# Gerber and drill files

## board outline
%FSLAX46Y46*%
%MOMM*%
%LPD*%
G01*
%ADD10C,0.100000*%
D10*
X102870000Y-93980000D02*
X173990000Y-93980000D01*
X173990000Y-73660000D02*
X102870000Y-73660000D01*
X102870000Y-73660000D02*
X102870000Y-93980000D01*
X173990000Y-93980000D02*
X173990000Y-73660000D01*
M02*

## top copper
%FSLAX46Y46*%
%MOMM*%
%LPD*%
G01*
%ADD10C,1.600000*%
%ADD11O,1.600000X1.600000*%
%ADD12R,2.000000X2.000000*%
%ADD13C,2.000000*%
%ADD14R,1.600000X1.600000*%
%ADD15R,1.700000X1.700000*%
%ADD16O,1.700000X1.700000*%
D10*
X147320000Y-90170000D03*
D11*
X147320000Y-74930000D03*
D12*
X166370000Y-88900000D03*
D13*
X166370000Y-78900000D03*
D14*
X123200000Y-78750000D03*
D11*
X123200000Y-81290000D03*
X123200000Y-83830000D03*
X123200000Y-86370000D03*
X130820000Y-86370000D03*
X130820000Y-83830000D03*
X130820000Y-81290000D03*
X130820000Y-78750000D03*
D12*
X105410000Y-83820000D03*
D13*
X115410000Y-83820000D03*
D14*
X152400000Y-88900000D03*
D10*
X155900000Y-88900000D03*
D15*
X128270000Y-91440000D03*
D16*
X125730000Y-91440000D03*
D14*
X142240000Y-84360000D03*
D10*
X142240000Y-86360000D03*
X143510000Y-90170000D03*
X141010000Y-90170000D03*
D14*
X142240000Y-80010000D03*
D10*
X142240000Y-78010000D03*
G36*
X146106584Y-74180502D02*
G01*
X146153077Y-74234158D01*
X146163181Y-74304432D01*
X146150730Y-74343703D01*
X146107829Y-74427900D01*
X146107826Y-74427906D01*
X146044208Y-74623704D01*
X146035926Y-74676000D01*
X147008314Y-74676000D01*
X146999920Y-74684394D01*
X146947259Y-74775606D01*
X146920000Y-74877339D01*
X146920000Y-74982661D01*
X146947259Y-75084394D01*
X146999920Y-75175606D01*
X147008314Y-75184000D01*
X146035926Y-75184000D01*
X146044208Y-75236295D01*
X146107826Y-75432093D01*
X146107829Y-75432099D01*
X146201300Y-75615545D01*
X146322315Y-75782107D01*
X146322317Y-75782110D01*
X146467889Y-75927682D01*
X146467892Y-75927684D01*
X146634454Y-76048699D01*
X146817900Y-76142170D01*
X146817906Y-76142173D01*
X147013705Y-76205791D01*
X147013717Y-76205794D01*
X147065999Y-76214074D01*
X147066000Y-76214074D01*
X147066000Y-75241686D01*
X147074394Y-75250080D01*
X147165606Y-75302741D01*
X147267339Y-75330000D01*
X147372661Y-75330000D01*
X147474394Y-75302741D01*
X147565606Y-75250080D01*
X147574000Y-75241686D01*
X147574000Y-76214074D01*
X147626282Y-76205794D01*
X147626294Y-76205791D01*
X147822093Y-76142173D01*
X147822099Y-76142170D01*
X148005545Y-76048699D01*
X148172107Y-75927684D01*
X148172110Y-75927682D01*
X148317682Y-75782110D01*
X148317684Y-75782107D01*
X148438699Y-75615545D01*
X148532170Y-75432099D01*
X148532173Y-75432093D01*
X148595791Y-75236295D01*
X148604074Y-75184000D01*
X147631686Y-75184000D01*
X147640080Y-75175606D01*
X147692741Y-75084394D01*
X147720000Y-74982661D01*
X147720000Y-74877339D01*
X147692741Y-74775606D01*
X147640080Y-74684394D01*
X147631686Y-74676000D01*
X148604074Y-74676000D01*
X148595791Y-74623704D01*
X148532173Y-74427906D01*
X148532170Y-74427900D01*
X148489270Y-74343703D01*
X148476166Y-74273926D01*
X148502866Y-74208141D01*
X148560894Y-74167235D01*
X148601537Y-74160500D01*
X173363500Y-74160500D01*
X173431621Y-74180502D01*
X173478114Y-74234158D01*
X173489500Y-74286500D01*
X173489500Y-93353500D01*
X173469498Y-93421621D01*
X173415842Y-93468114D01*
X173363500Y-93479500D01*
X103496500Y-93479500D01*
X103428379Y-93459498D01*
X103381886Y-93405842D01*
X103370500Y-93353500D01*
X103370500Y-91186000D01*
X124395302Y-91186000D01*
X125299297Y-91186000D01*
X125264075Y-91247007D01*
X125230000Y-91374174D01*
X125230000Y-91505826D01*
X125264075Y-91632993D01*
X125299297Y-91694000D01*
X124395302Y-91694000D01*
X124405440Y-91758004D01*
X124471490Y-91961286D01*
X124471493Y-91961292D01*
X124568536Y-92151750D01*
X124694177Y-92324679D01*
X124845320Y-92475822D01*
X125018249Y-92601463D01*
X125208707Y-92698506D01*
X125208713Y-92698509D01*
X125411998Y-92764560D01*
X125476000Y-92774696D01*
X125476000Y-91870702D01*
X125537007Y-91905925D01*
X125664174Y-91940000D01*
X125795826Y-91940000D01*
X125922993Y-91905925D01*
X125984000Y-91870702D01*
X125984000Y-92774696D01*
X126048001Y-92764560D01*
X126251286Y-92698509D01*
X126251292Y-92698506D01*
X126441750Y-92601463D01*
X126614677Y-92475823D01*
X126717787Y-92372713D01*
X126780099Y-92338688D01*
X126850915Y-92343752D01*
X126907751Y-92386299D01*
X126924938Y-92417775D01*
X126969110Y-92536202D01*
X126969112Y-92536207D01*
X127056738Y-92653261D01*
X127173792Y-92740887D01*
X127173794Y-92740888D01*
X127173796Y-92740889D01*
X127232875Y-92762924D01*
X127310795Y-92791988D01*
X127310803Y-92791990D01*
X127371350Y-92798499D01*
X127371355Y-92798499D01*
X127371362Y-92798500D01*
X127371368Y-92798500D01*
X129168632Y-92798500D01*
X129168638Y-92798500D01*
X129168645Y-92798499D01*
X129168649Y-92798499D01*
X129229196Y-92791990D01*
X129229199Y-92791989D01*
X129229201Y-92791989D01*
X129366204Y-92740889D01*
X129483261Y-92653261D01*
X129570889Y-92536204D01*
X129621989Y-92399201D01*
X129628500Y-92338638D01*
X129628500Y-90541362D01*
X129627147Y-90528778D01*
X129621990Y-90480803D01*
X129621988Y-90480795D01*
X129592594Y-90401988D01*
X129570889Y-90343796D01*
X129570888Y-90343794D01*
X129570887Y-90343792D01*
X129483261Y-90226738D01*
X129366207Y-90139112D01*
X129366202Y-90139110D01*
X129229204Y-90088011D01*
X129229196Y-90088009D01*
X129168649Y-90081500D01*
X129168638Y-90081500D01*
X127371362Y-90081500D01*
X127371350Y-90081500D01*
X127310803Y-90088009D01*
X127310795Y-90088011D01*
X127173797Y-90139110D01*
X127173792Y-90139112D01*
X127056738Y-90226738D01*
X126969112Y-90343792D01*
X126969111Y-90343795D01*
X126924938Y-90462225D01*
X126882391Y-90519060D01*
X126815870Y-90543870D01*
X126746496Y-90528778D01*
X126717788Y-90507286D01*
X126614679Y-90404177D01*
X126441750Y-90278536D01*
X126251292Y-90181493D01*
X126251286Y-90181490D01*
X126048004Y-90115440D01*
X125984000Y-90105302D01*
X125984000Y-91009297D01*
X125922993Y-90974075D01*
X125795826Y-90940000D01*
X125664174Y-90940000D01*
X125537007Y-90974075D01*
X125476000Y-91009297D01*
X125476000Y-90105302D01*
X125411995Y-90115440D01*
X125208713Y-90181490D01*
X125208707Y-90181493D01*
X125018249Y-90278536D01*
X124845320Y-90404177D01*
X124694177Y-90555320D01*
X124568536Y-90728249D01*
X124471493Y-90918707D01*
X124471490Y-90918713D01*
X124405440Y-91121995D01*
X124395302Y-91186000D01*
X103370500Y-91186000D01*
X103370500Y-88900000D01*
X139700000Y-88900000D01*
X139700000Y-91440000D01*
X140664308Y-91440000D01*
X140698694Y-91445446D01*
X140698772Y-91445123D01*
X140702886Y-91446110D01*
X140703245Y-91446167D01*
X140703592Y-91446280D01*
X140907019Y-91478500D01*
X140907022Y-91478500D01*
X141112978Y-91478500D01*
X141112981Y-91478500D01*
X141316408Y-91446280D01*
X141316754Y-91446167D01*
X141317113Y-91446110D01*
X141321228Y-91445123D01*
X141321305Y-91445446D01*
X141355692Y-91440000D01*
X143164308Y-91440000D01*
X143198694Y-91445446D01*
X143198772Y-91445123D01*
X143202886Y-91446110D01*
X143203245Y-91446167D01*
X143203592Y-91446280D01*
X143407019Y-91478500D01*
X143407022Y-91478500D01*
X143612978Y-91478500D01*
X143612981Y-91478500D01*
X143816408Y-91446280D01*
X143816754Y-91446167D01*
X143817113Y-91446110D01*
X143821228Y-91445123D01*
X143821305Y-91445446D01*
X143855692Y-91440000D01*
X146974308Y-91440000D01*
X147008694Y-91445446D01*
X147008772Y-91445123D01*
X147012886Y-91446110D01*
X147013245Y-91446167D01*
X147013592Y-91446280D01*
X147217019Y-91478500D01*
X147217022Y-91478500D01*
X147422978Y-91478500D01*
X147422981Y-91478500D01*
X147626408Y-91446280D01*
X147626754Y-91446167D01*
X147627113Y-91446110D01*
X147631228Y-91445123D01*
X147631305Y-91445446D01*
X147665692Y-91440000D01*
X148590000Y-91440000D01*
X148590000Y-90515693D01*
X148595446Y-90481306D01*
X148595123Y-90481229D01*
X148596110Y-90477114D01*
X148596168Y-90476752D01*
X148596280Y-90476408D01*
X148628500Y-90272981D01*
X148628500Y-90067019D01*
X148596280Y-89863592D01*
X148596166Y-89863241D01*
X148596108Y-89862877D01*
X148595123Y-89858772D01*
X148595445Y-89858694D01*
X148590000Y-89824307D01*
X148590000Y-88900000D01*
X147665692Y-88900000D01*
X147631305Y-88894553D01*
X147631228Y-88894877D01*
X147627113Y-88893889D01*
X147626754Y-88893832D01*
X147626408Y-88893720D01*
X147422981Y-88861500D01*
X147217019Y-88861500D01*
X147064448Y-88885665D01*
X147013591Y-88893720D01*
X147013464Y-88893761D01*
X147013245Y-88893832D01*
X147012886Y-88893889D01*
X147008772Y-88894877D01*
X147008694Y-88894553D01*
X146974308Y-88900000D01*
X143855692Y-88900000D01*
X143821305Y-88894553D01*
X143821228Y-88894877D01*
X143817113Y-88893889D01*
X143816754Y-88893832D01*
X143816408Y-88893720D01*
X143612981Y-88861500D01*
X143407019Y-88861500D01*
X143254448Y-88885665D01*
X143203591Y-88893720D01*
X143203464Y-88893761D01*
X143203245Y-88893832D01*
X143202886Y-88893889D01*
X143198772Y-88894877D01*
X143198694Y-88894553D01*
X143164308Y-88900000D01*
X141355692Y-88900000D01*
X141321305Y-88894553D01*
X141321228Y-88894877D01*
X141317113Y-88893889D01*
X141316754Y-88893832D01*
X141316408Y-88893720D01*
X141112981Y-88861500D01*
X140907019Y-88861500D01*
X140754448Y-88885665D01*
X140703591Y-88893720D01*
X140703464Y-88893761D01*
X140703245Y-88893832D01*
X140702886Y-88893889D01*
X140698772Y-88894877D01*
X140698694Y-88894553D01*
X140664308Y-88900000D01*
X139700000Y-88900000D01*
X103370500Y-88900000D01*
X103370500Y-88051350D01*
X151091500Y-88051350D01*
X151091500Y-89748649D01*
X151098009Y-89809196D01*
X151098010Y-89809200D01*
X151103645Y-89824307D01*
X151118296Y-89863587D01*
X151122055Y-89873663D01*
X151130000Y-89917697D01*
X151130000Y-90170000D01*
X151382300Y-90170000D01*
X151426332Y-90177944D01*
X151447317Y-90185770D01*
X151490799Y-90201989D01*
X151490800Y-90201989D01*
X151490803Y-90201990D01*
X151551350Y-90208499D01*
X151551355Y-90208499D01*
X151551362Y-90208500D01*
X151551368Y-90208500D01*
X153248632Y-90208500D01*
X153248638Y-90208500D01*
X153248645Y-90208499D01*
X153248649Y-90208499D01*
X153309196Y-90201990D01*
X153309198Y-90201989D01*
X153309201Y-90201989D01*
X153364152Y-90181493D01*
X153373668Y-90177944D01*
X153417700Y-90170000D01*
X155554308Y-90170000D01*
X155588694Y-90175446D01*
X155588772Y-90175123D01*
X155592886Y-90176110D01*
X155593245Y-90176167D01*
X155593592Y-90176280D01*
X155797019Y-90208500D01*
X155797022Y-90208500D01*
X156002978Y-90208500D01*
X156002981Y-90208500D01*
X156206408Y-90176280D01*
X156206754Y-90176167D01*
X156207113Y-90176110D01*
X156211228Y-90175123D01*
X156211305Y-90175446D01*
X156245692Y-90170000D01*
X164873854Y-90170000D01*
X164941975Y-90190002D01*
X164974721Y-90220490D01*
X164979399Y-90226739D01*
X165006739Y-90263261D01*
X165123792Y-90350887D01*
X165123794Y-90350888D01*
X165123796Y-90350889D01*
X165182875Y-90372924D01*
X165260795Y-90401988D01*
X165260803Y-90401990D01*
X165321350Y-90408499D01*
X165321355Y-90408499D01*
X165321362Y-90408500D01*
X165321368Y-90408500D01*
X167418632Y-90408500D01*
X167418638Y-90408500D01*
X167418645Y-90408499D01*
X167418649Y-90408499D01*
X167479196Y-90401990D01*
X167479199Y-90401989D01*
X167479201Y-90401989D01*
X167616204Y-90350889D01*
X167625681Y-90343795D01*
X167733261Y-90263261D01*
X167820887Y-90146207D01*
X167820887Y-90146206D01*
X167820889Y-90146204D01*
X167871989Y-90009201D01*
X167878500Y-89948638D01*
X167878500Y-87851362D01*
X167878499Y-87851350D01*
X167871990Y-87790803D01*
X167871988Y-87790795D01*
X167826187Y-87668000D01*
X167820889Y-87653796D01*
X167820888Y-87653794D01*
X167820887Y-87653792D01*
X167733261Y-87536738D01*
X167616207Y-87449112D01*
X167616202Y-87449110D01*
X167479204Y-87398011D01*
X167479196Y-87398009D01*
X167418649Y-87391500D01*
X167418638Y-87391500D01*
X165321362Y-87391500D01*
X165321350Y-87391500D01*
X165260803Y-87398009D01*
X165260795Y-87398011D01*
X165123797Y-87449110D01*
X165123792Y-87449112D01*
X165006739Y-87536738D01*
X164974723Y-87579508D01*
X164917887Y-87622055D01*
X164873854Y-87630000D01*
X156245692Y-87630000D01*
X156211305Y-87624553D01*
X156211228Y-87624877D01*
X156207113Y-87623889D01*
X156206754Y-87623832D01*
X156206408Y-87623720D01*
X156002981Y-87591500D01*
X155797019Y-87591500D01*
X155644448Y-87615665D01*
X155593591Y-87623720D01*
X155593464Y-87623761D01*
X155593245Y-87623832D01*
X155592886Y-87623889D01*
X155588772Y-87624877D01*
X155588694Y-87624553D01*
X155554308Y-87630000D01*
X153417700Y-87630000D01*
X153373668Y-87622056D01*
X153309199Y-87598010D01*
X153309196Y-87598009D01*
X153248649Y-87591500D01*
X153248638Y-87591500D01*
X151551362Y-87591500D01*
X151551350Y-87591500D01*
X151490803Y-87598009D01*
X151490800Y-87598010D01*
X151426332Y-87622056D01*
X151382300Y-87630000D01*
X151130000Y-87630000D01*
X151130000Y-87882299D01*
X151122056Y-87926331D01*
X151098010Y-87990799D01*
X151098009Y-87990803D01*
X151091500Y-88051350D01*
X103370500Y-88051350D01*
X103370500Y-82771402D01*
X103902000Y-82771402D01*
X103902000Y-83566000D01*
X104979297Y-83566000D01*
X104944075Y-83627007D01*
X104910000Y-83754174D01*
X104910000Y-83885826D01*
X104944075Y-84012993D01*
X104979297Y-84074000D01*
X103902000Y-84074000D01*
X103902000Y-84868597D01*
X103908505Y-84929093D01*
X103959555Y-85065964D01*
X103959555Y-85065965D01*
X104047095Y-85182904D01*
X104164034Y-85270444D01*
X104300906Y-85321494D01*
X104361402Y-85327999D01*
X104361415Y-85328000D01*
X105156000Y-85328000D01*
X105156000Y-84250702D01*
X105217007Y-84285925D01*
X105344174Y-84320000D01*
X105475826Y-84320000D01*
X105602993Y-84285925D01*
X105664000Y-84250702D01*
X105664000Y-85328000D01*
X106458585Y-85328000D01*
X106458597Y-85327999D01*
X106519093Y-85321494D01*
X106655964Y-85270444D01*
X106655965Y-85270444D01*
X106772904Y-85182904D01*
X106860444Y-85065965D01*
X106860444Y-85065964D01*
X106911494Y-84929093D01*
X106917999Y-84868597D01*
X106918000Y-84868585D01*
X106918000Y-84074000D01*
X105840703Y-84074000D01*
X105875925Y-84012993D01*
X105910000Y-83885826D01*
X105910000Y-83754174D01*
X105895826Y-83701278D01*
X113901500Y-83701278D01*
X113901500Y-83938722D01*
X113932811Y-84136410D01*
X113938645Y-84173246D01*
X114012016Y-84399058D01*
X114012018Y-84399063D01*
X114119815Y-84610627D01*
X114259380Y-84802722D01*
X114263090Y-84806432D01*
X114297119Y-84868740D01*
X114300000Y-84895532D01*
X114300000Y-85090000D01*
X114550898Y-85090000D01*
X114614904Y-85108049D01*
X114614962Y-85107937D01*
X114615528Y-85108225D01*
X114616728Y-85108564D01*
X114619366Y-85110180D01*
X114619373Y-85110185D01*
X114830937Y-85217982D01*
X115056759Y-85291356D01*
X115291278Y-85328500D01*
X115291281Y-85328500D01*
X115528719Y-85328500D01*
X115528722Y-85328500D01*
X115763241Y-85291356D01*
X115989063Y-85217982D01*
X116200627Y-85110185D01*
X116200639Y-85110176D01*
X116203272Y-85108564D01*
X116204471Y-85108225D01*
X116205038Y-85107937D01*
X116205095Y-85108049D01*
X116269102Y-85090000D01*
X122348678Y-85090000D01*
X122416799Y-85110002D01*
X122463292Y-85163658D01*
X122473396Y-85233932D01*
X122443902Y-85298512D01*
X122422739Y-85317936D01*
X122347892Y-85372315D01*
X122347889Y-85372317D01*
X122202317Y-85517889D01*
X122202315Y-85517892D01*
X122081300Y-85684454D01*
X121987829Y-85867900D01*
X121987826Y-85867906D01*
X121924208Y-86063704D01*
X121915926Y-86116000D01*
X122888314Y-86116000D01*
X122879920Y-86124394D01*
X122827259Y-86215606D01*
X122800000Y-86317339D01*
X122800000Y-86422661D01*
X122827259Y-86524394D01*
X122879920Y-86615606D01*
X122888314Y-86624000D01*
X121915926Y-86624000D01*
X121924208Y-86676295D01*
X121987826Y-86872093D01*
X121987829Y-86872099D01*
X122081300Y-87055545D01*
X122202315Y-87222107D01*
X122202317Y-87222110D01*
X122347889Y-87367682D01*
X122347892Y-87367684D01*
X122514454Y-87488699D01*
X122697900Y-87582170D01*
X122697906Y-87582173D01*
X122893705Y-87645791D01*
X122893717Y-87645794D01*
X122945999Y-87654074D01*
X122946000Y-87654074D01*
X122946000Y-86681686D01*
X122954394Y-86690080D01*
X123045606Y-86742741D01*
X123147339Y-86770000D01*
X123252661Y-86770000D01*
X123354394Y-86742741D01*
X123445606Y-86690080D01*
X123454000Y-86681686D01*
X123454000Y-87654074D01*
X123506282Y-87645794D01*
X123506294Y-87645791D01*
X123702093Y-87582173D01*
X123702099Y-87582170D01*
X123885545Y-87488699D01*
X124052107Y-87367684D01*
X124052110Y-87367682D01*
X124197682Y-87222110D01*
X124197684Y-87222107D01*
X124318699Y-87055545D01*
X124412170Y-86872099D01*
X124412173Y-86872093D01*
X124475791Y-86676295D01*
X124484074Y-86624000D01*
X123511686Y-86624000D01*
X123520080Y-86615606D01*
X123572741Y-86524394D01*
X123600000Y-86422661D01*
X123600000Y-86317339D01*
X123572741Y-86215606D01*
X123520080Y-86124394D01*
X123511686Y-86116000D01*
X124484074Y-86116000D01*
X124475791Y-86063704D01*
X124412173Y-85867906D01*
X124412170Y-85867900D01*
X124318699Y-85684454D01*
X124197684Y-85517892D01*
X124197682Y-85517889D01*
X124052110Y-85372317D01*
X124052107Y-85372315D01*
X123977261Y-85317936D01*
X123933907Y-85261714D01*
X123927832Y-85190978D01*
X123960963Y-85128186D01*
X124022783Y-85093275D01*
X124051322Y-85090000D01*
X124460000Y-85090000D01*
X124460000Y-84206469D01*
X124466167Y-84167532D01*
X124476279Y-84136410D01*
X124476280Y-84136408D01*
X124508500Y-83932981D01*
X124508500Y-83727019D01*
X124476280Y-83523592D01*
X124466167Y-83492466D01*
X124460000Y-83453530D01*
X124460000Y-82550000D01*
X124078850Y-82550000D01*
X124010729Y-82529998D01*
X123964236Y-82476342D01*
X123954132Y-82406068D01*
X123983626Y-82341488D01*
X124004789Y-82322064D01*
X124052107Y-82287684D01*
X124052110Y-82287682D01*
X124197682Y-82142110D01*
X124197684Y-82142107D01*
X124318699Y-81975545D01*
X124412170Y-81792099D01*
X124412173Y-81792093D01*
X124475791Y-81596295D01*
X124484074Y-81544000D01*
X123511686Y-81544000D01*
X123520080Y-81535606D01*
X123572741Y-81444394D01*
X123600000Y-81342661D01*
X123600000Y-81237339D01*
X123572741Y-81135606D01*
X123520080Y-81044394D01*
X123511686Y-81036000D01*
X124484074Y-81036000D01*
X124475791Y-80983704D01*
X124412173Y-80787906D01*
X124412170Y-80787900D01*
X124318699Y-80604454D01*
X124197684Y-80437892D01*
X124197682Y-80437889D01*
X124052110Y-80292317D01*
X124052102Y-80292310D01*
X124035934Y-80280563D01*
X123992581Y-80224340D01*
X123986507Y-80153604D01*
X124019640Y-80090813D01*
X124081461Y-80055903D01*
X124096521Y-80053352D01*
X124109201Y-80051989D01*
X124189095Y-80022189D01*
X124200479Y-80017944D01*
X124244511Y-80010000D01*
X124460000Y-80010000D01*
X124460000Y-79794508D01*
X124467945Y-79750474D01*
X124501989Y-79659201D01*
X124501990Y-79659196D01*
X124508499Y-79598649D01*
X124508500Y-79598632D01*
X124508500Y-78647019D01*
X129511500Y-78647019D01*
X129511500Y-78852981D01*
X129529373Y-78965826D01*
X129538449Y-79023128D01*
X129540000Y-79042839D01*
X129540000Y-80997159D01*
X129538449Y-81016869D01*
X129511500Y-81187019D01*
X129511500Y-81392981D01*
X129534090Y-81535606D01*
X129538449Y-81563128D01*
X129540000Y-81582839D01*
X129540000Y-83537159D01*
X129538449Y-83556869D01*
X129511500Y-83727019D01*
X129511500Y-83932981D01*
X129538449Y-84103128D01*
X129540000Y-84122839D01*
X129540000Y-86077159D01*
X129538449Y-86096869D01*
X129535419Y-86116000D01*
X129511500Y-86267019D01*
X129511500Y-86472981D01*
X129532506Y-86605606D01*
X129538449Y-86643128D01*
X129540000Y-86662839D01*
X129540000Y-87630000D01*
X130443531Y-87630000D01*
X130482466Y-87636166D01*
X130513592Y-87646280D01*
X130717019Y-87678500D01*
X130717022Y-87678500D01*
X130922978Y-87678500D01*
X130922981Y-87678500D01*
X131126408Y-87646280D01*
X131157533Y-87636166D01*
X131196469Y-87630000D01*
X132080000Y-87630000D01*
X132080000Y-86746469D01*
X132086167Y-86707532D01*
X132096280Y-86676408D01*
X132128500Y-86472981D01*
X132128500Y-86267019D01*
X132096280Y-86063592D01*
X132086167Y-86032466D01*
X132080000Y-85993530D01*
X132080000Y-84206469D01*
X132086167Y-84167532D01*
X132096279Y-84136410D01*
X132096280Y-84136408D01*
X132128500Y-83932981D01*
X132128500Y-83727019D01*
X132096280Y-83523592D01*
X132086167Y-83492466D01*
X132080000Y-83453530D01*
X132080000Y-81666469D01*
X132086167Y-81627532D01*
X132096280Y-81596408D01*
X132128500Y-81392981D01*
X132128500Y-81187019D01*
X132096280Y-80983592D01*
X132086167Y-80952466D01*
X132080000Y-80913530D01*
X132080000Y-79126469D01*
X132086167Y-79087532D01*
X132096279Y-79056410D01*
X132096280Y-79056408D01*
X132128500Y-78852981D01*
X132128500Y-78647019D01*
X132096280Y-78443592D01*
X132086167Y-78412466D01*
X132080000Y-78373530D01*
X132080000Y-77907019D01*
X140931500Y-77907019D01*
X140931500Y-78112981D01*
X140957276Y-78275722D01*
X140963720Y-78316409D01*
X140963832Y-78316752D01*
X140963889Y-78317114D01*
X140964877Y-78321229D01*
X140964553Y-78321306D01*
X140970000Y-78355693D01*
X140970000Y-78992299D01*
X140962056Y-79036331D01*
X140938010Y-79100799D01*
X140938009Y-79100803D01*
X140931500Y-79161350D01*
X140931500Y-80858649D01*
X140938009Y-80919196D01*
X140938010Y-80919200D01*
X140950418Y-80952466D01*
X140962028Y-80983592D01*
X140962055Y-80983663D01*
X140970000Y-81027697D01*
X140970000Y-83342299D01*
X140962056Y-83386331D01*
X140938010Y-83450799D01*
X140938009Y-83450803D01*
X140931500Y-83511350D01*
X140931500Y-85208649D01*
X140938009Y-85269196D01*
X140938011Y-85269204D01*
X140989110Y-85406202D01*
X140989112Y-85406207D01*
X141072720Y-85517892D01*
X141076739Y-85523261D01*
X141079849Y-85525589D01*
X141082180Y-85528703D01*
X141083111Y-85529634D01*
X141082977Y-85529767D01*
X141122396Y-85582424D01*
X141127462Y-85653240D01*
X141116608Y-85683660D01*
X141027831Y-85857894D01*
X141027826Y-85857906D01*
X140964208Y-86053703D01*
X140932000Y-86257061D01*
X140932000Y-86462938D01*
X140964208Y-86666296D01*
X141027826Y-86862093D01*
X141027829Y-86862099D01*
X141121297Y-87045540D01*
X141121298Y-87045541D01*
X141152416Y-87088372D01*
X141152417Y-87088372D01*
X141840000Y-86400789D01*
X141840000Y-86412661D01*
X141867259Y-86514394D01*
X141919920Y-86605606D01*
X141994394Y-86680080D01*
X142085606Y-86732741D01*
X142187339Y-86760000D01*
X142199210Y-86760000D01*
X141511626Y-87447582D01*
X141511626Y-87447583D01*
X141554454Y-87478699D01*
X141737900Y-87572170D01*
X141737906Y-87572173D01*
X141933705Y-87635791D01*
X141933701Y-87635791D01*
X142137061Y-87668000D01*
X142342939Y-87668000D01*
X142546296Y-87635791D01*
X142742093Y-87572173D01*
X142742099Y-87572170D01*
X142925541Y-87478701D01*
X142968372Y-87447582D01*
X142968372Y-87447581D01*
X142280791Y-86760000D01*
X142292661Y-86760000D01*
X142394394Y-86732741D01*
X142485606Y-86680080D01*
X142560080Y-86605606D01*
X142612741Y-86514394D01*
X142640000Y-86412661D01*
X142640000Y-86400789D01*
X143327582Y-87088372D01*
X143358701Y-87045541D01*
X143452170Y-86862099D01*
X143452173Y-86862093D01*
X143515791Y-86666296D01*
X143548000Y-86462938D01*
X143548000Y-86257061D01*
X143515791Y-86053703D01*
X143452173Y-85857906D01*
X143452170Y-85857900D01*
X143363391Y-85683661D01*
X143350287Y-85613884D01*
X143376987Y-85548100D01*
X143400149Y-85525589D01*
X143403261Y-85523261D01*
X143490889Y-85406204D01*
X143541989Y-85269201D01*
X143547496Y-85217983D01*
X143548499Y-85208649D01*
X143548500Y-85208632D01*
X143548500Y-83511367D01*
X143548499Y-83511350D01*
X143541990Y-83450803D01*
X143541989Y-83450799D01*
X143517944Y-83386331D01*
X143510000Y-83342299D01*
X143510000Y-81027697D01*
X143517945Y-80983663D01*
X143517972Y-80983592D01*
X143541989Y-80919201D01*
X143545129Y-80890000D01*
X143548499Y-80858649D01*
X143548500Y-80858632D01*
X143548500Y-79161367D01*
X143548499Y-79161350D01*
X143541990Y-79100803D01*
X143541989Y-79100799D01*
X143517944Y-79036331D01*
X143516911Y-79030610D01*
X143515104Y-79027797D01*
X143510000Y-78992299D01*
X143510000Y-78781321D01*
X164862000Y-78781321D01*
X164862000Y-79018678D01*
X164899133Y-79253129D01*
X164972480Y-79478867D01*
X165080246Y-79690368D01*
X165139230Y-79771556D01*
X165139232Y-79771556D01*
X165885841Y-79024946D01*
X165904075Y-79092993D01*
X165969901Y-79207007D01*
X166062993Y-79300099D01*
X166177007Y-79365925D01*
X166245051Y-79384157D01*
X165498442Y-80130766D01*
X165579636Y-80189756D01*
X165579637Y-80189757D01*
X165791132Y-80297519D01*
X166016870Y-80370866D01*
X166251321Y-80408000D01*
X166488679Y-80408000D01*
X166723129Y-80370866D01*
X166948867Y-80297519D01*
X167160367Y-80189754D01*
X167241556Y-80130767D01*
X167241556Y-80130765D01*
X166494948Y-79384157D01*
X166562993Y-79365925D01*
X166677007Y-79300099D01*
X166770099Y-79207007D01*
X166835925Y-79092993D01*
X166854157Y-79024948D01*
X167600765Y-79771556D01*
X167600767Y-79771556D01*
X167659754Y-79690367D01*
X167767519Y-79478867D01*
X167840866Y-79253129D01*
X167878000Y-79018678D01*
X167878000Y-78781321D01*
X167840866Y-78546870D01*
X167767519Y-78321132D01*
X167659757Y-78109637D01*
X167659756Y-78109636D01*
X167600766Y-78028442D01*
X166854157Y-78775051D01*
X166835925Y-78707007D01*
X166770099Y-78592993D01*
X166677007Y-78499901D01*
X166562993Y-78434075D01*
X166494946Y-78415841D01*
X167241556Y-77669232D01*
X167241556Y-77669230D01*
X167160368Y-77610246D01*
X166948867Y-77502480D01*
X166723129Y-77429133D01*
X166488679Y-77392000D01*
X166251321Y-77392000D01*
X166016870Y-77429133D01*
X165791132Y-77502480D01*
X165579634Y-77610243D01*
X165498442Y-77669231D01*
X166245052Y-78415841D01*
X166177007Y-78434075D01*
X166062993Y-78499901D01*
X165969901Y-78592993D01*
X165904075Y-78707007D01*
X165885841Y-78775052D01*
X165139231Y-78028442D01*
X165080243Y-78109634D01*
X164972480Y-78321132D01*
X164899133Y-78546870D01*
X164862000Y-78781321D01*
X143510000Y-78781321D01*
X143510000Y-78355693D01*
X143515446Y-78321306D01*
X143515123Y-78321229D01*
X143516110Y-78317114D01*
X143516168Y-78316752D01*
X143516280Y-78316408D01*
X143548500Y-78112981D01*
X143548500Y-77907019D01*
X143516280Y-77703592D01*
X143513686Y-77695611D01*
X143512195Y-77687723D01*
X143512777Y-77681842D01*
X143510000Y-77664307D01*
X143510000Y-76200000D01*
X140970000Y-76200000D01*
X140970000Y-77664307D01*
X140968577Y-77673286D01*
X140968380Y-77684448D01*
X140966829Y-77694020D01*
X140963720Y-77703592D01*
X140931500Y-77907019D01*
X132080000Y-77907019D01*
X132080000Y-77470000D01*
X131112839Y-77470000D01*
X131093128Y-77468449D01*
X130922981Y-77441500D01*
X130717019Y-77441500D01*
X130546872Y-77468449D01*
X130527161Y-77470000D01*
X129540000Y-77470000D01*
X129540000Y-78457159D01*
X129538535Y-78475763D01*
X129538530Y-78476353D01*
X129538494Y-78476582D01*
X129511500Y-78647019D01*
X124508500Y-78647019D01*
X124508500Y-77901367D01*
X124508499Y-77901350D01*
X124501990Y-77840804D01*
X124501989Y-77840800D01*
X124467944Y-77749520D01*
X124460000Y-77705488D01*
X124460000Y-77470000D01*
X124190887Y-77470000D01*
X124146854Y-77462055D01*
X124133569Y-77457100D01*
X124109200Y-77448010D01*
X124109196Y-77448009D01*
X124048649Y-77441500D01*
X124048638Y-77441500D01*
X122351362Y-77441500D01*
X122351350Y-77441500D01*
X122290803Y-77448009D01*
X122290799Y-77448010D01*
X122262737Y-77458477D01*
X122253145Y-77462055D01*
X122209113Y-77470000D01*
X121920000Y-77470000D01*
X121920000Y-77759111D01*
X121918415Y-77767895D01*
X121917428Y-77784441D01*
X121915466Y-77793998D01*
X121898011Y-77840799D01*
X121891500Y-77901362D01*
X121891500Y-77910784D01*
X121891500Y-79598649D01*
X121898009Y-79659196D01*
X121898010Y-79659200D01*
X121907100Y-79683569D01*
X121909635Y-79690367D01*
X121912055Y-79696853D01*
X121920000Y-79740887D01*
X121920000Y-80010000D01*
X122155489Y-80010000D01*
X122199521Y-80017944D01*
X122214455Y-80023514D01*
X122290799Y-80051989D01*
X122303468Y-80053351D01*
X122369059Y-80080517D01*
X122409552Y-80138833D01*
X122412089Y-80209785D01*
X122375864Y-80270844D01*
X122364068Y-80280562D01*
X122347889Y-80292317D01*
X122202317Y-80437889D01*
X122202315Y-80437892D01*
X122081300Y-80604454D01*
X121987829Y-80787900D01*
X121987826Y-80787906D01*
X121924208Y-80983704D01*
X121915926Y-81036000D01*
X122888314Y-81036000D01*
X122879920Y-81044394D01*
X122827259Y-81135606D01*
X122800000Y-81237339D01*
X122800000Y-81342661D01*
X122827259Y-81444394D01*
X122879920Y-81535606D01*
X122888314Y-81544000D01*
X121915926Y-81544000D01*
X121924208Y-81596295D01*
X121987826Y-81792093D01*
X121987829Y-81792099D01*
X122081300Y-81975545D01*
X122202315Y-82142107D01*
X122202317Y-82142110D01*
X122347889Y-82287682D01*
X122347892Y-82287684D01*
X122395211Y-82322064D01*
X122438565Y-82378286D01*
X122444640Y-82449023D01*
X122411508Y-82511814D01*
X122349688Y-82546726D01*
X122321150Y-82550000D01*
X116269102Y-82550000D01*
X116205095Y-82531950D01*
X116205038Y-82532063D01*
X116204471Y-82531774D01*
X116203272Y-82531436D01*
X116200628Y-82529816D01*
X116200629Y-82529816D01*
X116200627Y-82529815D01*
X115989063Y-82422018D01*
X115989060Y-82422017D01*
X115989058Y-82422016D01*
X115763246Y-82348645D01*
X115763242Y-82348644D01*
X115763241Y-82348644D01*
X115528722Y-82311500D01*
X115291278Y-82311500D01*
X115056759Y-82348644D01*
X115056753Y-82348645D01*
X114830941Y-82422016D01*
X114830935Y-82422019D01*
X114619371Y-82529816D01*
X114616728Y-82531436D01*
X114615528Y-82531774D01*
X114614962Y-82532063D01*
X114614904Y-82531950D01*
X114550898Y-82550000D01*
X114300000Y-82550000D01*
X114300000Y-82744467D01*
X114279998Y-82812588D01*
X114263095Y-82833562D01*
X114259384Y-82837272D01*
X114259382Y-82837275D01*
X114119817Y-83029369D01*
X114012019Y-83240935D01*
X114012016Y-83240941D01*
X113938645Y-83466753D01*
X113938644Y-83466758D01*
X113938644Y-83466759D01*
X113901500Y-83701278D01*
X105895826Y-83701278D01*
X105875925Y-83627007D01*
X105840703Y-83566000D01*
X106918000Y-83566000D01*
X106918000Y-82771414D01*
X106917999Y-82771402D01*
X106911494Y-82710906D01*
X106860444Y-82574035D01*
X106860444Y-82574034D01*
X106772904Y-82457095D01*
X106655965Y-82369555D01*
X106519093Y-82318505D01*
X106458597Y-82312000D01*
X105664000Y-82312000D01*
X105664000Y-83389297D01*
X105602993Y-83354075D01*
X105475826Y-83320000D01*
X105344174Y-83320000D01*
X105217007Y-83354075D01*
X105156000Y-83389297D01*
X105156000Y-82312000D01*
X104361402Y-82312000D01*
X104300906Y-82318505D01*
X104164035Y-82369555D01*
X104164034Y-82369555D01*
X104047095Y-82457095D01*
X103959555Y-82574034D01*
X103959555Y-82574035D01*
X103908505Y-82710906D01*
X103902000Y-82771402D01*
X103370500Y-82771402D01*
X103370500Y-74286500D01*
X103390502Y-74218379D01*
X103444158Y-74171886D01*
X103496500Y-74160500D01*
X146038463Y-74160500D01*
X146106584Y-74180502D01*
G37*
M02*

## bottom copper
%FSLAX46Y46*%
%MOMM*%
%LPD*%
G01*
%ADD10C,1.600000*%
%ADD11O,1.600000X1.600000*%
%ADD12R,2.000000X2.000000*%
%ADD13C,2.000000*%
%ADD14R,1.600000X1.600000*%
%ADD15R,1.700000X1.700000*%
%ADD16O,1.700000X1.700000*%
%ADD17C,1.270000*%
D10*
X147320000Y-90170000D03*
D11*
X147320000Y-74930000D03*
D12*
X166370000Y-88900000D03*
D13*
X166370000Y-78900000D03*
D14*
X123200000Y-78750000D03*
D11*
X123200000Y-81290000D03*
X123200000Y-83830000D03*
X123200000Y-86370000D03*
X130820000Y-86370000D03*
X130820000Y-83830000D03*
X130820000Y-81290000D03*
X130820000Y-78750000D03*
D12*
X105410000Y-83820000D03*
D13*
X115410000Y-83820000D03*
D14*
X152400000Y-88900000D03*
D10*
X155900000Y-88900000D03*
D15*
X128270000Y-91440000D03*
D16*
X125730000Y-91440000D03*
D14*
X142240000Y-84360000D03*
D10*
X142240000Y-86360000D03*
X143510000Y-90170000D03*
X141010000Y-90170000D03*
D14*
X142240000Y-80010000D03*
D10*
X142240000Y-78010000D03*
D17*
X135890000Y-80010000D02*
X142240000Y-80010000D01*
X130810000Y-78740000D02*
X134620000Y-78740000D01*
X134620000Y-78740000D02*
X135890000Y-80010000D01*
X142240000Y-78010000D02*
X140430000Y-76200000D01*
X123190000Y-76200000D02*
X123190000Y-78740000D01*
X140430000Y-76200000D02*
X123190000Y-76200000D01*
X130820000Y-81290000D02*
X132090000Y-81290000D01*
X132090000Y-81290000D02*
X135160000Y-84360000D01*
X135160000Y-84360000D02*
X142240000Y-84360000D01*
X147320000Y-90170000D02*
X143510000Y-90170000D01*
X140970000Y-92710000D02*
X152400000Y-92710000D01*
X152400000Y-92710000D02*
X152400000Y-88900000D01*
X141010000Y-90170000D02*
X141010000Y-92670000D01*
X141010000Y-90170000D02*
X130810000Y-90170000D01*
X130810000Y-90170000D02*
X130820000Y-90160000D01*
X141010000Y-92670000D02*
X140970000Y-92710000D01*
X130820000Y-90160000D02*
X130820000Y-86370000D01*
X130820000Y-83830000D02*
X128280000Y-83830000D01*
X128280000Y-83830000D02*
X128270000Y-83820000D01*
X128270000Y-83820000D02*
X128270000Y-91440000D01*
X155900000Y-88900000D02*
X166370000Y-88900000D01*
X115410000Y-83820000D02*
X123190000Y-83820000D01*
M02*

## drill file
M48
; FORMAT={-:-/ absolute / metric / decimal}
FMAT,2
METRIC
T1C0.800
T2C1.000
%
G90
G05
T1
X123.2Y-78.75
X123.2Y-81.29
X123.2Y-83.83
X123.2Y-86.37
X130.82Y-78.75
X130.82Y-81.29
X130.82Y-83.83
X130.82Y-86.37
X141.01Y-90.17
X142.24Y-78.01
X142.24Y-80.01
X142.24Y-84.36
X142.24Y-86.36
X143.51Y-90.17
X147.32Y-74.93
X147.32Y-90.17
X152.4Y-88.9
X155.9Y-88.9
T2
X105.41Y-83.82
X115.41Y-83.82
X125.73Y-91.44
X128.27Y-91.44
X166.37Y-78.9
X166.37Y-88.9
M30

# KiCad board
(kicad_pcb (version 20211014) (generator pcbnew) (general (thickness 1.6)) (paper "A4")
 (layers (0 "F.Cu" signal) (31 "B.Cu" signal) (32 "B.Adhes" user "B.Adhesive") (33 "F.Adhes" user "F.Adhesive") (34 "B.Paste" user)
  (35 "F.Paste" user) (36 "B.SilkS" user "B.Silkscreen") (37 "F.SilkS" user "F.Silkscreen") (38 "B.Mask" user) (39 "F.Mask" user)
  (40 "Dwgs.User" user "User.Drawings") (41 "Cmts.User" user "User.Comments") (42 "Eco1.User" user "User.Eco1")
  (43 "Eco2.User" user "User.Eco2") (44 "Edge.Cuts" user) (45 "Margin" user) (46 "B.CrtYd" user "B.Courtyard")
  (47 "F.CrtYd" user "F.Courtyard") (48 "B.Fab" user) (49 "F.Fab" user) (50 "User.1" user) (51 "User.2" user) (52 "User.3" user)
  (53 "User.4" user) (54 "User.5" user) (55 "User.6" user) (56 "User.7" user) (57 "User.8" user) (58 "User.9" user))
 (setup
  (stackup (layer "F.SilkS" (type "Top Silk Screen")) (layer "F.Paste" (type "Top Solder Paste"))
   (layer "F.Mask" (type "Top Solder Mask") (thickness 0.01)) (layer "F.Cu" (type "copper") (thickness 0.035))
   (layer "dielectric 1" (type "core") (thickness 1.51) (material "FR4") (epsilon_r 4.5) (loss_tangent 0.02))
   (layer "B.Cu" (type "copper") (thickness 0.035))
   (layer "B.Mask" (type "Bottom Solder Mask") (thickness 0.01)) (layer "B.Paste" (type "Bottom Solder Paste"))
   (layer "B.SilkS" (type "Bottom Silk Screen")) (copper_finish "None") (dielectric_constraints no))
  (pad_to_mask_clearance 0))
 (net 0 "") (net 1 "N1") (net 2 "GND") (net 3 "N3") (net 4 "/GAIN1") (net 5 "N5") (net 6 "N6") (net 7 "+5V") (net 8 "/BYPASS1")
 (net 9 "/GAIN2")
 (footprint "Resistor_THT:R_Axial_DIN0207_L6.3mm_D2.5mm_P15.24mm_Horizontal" (layer "F.Cu") (at 147.32 90.17 90)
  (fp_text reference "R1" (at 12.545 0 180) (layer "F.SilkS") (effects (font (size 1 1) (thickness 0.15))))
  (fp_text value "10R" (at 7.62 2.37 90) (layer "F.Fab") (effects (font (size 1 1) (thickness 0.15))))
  (pad "1" thru_hole circle (at 0 0 90) (size 1.6 1.6) (drill 0.8) (layers *.Cu *.Mask) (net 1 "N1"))
  (pad "2" thru_hole oval (at 15.24 0 90) (size 1.6 1.6) (drill 0.8) (layers *.Cu *.Mask) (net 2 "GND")))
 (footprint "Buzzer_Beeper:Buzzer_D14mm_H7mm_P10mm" (layer "F.Cu") (at 166.37 88.9 90)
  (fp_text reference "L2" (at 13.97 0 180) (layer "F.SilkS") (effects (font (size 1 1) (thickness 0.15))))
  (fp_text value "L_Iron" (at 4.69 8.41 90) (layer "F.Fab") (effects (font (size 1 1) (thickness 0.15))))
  (pad "1" thru_hole rect (at 0 0 90) (size 2 2) (drill 1) (layers *.Cu *.Mask) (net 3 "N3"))
  (pad "2" thru_hole circle (at 10 0 90) (size 2 2) (drill 1) (layers *.Cu *.Mask) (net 2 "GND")))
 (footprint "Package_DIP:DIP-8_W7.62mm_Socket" (layer "F.Cu") (at 123.2 78.75)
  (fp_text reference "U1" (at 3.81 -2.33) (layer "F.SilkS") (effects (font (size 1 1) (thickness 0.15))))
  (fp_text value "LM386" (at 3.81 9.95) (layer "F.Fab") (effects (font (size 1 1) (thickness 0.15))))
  (pad "1" thru_hole rect (at 0 0) (size 1.6 1.6) (drill 0.8) (layers *.Cu *.Mask) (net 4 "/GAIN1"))
  (pad "2" thru_hole oval (at 0 2.54) (size 1.6 1.6) (drill 0.8) (layers *.Cu *.Mask) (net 2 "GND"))
  (pad "3" thru_hole oval (at 0 5.08) (size 1.6 1.6) (drill 0.8) (layers *.Cu *.Mask) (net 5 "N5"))
  (pad "4" thru_hole oval (at 0 7.62) (size 1.6 1.6) (drill 0.8) (layers *.Cu *.Mask) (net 2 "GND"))
  (pad "5" thru_hole oval (at 7.62 7.62) (size 1.6 1.6) (drill 0.8) (layers *.Cu *.Mask) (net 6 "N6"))
  (pad "6" thru_hole oval (at 7.62 5.08) (size 1.6 1.6) (drill 0.8) (layers *.Cu *.Mask) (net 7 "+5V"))
  (pad "7" thru_hole oval (at 7.62 2.54) (size 1.6 1.6) (drill 0.8) (layers *.Cu *.Mask) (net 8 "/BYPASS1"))
  (pad "8" thru_hole oval (at 7.62 0) (size 1.6 1.6) (drill 0.8) (layers *.Cu *.Mask) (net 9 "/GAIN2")))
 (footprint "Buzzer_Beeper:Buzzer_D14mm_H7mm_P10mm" (layer "F.Cu") (at 105.41 83.82)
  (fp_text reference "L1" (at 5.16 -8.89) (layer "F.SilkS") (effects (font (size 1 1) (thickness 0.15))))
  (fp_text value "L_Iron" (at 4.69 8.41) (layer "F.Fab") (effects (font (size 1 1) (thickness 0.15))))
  (pad "1" thru_hole rect (at 0 0) (size 2 2) (drill 1) (layers *.Cu *.Mask) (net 2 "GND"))
  (pad "2" thru_hole circle (at 10 0) (size 2 2) (drill 1) (layers *.Cu *.Mask) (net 5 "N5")))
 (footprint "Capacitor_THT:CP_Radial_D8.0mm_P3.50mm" (layer "F.Cu") (at 152.4 88.9)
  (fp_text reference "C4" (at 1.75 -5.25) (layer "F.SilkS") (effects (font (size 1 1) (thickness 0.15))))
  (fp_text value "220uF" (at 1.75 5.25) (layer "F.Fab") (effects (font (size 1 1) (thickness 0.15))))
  (pad "1" thru_hole rect (at 0 0) (size 1.6 1.6) (drill 0.8) (layers *.Cu *.Mask) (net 6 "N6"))
  (pad "2" thru_hole circle (at 3.5 0) (size 1.6 1.6) (drill 0.8) (layers *.Cu *.Mask) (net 3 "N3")))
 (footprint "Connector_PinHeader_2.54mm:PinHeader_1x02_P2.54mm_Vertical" (layer "F.Cu") (at 128.27 91.44 -90)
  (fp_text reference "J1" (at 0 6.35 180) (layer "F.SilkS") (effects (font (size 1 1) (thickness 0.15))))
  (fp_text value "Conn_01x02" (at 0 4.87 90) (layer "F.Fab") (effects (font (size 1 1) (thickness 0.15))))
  (pad "1" thru_hole rect (at 0 0 270) (size 1.7 1.7) (drill 1) (layers *.Cu *.Mask) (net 7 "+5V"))
  (pad "2" thru_hole oval (at 0 2.54 270) (size 1.7 1.7) (drill 1) (layers *.Cu *.Mask) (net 2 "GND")))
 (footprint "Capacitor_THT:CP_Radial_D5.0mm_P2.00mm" (layer "F.Cu") (at 142.24 84.36 -90)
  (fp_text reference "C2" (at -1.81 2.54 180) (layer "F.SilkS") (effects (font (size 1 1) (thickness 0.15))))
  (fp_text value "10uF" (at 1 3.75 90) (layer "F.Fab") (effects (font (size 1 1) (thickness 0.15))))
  (pad "1" thru_hole rect (at 0 0 270) (size 1.6 1.6) (drill 0.8) (layers *.Cu *.Mask) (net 8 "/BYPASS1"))
  (pad "2" thru_hole circle (at 2 0 270) (size 1.6 1.6) (drill 0.8) (layers *.Cu *.Mask) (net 2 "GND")))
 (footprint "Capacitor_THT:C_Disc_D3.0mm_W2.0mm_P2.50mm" (layer "F.Cu") (at 143.51 90.17 180)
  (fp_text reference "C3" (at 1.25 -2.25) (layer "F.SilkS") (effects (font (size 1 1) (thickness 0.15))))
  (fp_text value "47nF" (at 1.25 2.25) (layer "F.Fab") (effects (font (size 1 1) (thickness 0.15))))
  (pad "1" thru_hole circle (at 0 0 180) (size 1.6 1.6) (drill 0.8) (layers *.Cu *.Mask) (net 1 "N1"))
  (pad "2" thru_hole circle (at 2.5 0 180) (size 1.6 1.6) (drill 0.8) (layers *.Cu *.Mask) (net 6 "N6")))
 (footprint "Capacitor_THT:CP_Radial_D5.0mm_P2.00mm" (layer "F.Cu") (at 142.24 80.01 90)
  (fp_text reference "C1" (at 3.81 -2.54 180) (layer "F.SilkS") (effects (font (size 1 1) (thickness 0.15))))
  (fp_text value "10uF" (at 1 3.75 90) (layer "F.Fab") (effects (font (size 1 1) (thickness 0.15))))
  (pad "1" thru_hole rect (at 0 0 90) (size 1.6 1.6) (drill 0.8) (layers *.Cu *.Mask) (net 9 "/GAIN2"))
  (pad "2" thru_hole circle (at 2 0 90) (size 1.6 1.6) (drill 0.8) (layers *.Cu *.Mask) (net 4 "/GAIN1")))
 (gr_line (start 102.87 93.98) (end 173.99 93.98) (layer "Edge.Cuts") (width 0.1))
 (gr_line (start 173.99 73.66) (end 102.87 73.66) (layer "Edge.Cuts") (width 0.1))
 (gr_line (start 102.87 73.66) (end 102.87 93.98) (layer "Edge.Cuts") (width 0.1))
 (gr_line (start 173.99 93.98) (end 173.99 73.66) (layer "Edge.Cuts") (width 0.1))
 (segment (start 135.89 80.01) (end 142.24 80.01) (width 1.27) (layer "B.Cu") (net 9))
 (segment (start 130.81 78.74) (end 134.62 78.74) (width 1.27) (layer "B.Cu") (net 9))
 (segment (start 134.62 78.74) (end 135.89 80.01) (width 1.27) (layer "B.Cu") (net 9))
 (segment (start 142.24 78.01) (end 140.43 76.2) (width 1.27) (layer "B.Cu") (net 4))
 (segment (start 123.19 76.2) (end 123.19 78.74) (width 1.27) (layer "B.Cu") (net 4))
 (segment (start 140.43 76.2) (end 123.19 76.2) (width 1.27) (layer "B.Cu") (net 4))
 (segment (start 130.82 81.29) (end 132.09 81.29) (width 1.27) (layer "B.Cu") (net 8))
 (segment (start 132.09 81.29) (end 135.16 84.36) (width 1.27) (layer "B.Cu") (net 8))
 (segment (start 135.16 84.36) (end 142.24 84.36) (width 1.27) (layer "B.Cu") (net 8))
 (segment (start 147.32 90.17) (end 143.51 90.17) (width 1.27) (layer "B.Cu") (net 1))
 (segment (start 140.97 92.71) (end 152.4 92.71) (width 1.27) (layer "B.Cu") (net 6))
 (segment (start 152.4 92.71) (end 152.4 88.9) (width 1.27) (layer "B.Cu") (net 6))
 (segment (start 141.01 90.17) (end 141.01 92.67) (width 1.27) (layer "B.Cu") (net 6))
 (segment (start 141.01 90.17) (end 130.81 90.17) (width 1.27) (layer "B.Cu") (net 6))
 (segment (start 130.81 90.17) (end 130.82 90.16) (width 1.27) (layer "B.Cu") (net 6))
 (segment (start 141.01 92.67) (end 140.97 92.71) (width 1.27) (layer "B.Cu") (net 6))
 (segment (start 130.82 90.16) (end 130.82 86.37) (width 1.27) (layer "B.Cu") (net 6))
 (segment (start 130.82 83.83) (end 128.28 83.83) (width 1.27) (layer "B.Cu") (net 7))
 (segment (start 128.28 83.83) (end 128.27 83.82) (width 1.27) (layer "B.Cu") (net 7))
 (segment (start 128.27 83.82) (end 128.27 91.44) (width 1.27) (layer "B.Cu") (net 7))
 (segment (start 155.9 88.9) (end 166.37 88.9) (width 1.27) (layer "B.Cu") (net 3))
 (segment (start 115.41 83.82) (end 123.19 83.82) (width 1.27) (layer "B.Cu") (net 5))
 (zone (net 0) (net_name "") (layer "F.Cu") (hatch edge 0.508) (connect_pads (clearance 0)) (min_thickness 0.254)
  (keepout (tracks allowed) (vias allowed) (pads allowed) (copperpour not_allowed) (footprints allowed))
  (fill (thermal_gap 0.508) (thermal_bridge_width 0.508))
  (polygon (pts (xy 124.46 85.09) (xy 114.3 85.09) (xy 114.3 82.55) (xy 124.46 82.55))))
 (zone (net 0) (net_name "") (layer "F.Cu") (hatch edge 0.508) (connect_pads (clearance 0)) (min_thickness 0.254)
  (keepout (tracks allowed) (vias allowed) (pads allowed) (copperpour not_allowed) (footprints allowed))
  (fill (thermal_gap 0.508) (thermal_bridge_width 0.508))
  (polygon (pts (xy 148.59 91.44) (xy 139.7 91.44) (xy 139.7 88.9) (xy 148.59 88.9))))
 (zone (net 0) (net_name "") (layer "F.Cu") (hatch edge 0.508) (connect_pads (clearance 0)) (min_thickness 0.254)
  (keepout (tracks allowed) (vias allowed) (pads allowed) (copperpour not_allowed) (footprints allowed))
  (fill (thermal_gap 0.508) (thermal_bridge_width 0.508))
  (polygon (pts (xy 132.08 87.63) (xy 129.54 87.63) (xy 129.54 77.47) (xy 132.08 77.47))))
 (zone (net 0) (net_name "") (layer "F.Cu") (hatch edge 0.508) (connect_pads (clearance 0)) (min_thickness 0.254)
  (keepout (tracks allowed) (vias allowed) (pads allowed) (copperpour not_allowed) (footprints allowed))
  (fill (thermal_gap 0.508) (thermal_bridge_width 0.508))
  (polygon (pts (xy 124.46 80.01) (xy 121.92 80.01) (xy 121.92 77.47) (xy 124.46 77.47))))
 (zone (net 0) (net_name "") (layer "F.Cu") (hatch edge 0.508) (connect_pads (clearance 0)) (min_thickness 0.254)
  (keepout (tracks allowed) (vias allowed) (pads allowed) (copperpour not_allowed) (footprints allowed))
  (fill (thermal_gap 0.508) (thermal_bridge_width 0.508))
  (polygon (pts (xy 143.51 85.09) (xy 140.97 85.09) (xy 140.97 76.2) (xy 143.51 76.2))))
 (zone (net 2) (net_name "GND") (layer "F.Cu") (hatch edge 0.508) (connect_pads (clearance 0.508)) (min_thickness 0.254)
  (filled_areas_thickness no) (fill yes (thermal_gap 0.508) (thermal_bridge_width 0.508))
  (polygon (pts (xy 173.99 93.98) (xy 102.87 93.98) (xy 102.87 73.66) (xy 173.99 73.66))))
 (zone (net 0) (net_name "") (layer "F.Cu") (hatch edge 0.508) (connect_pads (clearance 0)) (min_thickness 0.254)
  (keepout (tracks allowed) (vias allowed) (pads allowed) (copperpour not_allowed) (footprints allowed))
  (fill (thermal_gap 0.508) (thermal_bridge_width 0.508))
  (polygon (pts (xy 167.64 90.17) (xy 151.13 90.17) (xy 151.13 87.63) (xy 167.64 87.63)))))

